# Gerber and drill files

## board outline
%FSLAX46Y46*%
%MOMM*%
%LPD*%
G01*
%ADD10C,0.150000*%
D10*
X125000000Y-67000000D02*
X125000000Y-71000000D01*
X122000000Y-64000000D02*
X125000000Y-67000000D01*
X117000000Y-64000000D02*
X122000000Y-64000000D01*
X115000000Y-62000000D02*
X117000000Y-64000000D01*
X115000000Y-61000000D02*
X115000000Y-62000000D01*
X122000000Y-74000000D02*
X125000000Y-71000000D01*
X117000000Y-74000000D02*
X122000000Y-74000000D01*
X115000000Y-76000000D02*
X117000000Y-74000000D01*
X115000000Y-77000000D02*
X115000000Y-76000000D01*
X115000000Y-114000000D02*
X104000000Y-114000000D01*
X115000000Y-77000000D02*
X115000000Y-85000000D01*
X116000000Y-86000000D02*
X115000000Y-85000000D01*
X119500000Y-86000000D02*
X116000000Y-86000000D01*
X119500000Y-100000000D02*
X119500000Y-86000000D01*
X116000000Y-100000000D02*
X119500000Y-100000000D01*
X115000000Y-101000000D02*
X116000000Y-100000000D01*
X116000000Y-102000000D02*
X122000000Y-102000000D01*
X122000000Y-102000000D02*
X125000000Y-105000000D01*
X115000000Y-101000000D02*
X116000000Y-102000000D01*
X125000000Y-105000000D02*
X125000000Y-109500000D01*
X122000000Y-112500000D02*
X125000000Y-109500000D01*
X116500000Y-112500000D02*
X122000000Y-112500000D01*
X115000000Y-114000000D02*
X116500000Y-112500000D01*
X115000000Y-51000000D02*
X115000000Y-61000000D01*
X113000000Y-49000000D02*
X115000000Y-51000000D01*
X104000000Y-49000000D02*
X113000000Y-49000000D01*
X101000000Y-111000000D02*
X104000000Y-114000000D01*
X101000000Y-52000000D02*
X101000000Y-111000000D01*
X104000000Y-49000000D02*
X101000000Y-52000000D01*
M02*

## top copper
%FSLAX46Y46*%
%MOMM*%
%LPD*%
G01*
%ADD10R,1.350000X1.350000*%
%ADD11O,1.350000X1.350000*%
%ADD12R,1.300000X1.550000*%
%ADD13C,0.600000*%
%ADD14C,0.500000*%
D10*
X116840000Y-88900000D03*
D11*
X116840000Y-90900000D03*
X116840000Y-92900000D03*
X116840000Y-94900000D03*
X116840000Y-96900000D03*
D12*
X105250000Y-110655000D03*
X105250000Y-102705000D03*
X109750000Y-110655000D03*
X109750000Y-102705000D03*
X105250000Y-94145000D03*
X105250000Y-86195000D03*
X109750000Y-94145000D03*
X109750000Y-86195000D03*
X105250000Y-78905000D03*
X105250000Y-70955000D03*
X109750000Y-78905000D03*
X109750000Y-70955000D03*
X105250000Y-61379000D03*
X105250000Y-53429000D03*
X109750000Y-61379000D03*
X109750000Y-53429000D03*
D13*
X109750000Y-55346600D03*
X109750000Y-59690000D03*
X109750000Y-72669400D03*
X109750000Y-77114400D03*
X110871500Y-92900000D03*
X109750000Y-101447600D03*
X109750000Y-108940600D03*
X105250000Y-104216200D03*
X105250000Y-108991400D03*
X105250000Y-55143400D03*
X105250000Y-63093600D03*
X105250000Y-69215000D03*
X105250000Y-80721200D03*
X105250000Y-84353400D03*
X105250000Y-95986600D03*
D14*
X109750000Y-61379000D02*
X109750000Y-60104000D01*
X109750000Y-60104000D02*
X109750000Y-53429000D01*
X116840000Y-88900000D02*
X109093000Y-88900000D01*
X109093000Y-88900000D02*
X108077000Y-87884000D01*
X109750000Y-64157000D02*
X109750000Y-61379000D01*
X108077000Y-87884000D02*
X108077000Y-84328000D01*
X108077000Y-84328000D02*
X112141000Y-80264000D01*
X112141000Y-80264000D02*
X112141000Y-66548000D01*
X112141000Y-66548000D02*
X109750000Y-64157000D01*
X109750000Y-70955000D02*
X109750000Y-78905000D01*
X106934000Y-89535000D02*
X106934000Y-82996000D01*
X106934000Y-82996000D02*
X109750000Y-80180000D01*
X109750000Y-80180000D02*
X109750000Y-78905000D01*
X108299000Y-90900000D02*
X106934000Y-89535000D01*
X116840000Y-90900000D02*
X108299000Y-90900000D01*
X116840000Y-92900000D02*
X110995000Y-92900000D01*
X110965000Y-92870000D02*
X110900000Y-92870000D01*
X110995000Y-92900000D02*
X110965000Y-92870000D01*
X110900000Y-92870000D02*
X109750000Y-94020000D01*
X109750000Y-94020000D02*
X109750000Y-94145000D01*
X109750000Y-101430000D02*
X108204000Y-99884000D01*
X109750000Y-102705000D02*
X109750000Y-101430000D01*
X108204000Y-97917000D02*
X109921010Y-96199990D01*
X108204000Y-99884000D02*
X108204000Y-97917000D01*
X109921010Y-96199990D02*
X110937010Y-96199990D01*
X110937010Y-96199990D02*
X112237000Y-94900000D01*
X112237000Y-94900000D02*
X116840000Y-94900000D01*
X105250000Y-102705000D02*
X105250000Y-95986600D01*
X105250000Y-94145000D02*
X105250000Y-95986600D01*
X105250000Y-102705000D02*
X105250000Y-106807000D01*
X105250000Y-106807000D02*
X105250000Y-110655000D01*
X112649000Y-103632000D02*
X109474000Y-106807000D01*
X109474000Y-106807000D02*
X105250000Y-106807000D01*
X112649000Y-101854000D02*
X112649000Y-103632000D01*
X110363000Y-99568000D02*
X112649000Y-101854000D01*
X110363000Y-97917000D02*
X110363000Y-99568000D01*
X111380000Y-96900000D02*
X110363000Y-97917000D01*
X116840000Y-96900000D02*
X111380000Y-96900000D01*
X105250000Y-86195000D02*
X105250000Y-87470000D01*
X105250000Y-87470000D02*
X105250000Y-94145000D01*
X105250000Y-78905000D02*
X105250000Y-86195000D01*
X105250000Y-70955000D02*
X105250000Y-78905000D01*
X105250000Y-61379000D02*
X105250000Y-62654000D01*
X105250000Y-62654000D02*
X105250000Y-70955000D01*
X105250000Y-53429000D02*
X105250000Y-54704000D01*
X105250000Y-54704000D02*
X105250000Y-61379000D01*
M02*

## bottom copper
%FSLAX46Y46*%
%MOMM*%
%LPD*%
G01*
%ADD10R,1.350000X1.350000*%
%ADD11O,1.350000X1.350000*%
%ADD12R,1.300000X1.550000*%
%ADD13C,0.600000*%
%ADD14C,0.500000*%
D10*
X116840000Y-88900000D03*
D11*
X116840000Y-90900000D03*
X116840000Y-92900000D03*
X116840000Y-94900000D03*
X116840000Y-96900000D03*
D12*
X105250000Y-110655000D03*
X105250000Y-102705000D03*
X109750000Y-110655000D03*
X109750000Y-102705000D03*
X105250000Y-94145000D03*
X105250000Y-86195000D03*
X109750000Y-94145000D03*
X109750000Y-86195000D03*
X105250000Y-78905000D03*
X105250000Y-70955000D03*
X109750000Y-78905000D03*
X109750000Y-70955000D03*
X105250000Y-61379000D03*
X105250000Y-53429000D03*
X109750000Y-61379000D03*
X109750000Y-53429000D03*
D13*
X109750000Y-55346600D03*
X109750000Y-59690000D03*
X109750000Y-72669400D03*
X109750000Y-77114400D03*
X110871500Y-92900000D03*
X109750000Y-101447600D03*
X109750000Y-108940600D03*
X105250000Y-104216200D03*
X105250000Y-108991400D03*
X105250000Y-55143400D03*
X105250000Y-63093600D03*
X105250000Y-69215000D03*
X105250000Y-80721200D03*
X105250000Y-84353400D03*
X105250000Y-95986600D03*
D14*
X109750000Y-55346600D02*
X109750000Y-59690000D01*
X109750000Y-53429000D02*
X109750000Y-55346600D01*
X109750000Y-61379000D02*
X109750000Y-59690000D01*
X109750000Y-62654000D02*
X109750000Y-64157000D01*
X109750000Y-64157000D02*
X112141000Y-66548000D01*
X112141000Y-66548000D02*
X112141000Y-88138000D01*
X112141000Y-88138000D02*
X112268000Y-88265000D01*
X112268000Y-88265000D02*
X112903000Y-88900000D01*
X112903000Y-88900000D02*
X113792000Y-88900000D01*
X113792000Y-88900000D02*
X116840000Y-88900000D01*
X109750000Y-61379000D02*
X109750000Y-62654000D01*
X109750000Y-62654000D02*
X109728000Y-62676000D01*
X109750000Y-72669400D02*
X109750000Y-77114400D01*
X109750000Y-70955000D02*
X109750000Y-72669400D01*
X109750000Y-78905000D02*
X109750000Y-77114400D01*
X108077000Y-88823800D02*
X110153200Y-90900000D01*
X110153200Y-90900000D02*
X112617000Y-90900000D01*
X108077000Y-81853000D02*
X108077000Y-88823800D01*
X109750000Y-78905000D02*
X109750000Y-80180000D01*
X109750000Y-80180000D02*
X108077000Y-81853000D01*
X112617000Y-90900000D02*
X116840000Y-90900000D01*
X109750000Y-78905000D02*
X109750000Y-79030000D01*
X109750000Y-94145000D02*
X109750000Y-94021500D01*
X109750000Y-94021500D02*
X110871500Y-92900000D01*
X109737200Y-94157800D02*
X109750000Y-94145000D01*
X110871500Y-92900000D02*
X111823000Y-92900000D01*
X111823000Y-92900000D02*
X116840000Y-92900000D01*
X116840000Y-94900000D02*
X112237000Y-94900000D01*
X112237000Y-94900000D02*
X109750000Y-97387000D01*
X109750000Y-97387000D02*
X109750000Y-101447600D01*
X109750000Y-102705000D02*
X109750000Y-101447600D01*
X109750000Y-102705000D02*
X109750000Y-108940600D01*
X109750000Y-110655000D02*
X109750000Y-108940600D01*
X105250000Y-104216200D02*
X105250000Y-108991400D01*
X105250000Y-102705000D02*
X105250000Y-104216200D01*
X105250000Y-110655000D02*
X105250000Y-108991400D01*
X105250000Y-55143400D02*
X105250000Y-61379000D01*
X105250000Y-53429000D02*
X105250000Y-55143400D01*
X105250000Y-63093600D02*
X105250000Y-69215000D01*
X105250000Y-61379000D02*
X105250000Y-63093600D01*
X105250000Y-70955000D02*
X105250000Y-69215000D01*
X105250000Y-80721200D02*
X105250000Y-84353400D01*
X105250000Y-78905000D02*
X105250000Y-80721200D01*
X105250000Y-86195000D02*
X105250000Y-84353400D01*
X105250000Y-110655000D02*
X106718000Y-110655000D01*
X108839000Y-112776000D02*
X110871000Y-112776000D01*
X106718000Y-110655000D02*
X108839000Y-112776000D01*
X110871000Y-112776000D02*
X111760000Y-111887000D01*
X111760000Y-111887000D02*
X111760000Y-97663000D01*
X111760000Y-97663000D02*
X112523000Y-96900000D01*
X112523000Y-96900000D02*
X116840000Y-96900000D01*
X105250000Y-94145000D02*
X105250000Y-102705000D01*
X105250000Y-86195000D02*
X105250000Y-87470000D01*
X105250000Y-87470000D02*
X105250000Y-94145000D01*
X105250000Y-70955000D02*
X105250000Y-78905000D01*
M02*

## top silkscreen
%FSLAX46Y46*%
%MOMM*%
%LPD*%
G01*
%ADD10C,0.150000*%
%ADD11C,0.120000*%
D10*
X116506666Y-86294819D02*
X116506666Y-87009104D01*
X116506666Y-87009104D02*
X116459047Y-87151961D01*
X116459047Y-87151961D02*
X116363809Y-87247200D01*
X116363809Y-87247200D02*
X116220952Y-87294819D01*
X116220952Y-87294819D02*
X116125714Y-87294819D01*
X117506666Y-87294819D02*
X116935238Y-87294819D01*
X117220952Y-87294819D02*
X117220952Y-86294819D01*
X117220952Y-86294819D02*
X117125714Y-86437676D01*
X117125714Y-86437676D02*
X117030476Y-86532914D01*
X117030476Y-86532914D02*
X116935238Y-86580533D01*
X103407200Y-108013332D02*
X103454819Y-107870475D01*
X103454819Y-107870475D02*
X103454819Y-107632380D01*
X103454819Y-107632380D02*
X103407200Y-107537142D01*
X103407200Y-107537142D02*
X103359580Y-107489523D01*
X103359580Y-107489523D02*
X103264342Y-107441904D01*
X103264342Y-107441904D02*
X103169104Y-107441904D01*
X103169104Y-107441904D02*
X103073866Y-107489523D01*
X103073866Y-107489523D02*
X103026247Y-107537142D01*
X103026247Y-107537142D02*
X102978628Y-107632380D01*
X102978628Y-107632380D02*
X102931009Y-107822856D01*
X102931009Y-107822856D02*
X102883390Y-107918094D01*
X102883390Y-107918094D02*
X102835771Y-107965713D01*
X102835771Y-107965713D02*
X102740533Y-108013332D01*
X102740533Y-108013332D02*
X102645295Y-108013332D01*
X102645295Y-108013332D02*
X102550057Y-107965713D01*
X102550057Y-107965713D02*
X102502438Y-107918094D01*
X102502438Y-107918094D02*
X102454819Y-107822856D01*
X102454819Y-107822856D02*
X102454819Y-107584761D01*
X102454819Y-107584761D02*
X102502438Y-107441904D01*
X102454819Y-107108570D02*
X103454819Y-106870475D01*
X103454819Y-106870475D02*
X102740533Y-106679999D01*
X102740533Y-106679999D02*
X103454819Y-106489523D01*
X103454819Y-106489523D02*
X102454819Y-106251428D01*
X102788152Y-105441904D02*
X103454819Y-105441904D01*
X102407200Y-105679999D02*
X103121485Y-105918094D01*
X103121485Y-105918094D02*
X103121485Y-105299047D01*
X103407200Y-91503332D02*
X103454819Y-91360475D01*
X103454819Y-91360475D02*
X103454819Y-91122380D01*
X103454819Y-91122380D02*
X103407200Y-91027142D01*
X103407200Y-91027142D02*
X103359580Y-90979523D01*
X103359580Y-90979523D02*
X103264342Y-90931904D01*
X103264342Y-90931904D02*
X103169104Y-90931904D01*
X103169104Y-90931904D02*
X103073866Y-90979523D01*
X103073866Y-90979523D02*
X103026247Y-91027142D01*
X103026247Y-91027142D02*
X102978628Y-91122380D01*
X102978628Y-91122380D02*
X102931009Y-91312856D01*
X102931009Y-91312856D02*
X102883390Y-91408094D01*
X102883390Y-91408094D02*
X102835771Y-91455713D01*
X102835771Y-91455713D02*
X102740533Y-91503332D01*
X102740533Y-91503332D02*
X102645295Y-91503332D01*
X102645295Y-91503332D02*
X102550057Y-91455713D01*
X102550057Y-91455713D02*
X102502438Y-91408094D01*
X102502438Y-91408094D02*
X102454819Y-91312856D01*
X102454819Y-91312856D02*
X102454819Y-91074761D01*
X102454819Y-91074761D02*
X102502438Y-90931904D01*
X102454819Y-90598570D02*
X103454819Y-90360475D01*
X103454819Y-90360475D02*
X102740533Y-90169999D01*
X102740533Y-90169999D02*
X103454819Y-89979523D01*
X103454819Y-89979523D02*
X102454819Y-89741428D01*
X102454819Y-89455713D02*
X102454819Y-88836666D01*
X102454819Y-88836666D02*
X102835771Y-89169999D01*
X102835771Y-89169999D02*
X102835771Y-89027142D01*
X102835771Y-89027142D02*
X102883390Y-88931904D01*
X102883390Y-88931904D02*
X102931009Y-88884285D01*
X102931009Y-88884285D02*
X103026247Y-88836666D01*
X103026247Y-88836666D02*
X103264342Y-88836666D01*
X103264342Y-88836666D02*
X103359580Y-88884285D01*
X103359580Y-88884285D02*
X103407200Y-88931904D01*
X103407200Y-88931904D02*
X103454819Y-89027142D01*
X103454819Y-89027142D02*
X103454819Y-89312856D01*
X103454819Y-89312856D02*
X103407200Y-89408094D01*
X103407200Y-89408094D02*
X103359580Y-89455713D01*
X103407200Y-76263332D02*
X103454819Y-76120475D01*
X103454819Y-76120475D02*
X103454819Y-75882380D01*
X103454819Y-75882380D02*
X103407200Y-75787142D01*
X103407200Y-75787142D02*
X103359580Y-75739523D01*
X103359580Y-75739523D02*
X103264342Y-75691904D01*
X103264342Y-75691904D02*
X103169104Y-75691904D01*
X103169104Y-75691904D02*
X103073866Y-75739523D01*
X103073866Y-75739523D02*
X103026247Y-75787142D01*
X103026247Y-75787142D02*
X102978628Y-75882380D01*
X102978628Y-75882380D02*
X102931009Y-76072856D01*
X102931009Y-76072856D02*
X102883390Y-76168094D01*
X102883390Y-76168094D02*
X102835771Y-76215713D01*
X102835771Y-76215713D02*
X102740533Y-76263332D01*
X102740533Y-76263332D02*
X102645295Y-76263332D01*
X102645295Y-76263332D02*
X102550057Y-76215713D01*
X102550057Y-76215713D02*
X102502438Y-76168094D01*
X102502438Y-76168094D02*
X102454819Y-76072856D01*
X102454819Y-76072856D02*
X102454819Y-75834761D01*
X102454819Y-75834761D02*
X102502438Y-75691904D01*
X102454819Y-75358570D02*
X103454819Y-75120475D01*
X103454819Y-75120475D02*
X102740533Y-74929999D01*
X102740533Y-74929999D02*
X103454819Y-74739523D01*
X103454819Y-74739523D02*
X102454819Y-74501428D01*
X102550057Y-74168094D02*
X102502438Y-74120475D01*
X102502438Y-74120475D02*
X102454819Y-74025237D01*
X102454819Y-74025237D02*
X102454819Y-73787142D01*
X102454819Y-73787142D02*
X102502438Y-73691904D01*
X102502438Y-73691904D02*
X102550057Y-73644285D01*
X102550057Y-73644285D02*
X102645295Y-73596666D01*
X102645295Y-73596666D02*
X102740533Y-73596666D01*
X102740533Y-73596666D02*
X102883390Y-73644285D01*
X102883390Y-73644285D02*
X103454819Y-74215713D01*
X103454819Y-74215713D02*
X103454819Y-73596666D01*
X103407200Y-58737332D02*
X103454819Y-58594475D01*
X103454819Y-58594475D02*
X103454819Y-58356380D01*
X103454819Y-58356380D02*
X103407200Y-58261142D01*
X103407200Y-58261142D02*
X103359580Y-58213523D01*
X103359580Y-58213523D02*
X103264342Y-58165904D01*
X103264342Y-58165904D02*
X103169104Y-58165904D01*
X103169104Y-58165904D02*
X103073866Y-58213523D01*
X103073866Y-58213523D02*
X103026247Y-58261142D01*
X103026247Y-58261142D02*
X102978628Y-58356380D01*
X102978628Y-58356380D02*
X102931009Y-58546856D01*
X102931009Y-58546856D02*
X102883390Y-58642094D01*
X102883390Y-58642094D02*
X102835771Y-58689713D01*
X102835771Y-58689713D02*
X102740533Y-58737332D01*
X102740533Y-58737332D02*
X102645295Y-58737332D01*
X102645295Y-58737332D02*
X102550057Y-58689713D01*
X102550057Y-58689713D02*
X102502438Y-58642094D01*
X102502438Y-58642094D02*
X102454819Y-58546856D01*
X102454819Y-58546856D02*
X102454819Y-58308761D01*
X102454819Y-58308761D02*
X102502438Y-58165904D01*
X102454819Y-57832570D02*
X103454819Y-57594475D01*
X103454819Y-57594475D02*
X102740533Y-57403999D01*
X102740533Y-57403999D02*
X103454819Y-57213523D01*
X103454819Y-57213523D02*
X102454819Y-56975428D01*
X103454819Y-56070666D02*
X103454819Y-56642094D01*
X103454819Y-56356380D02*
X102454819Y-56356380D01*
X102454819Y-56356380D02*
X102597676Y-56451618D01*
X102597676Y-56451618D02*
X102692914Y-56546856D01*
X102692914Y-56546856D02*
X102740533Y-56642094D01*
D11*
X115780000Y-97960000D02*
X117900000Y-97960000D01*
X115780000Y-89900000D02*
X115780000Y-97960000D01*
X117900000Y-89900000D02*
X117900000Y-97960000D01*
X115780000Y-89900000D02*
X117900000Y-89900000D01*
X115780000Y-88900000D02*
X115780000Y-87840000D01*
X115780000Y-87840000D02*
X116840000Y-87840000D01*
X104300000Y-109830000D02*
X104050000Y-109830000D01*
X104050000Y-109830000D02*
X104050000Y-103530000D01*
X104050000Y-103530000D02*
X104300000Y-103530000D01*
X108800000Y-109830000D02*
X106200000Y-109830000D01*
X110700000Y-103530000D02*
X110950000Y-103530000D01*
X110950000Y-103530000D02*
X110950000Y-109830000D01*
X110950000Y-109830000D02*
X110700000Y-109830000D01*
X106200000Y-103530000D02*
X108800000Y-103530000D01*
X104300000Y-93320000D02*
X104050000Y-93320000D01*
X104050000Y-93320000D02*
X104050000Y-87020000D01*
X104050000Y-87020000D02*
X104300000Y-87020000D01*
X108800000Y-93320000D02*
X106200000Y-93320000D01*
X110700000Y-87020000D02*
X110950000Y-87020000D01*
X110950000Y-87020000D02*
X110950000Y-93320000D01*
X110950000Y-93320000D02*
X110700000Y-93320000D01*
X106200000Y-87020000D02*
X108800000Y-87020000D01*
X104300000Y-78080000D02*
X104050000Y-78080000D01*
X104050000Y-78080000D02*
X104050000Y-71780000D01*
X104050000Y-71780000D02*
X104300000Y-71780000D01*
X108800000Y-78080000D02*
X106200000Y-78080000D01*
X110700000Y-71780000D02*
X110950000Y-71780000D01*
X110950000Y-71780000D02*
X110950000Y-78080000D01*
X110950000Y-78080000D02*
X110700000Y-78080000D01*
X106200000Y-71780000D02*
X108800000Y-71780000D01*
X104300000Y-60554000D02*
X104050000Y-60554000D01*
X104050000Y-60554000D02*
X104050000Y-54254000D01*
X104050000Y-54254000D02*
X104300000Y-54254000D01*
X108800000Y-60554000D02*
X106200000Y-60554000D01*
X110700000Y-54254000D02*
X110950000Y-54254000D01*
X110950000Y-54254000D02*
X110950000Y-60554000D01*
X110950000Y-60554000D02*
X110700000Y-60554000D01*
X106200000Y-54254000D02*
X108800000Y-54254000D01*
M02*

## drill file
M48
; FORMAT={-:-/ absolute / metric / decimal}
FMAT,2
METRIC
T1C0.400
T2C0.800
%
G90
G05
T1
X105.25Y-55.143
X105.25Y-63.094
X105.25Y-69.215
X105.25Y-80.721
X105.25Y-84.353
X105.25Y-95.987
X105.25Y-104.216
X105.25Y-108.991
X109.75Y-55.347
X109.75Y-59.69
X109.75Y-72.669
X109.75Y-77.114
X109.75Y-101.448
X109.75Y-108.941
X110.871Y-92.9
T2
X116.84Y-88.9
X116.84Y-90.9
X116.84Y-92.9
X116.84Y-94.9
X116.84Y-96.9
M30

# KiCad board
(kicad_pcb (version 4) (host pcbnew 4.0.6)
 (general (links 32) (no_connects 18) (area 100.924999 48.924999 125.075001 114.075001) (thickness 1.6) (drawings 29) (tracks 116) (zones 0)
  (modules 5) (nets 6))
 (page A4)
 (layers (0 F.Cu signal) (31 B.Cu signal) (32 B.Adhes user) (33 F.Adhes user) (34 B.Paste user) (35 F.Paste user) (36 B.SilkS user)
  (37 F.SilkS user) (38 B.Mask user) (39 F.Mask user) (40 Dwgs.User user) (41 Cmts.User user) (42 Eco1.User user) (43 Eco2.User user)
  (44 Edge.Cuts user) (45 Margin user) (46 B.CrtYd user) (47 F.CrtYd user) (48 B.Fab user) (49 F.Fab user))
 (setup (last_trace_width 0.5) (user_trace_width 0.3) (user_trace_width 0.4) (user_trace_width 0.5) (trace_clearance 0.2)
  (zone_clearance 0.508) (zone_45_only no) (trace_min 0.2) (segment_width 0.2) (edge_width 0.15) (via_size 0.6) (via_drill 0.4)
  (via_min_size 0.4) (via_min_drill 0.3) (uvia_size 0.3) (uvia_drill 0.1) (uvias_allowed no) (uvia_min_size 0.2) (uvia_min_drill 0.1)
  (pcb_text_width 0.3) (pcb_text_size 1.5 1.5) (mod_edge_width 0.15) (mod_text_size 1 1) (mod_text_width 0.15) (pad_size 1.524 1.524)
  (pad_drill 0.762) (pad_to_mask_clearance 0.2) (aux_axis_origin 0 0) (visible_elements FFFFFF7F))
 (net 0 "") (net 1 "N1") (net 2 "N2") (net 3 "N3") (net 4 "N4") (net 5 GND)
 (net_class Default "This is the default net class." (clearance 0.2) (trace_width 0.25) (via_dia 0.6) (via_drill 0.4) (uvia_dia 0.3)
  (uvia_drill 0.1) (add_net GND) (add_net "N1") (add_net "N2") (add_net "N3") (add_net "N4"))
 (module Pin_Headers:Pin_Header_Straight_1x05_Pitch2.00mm (layer F.Cu) (at 116.84 88.9)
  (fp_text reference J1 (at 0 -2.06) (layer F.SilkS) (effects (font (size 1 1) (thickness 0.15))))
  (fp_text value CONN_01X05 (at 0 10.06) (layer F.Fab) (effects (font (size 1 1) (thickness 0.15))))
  (fp_line (start -1.06 9.06) (end 1.06 9.06) (layer F.SilkS) (width 0.12))
  (fp_line (start -1.06 1) (end -1.06 9.06) (layer F.SilkS) (width 0.12))
  (fp_line (start 1.06 1) (end 1.06 9.06) (layer F.SilkS) (width 0.12))
  (fp_line (start -1.06 1) (end 1.06 1) (layer F.SilkS) (width 0.12))
  (fp_line (start -1.06 0) (end -1.06 -1.06) (layer F.SilkS) (width 0.12))
  (fp_line (start -1.06 -1.06) (end 0 -1.06) (layer F.SilkS) (width 0.12))
  (pad 1 thru_hole rect (at 0 0) (size 1.35 1.35) (drill 0.8) (layers *.Cu *.Mask) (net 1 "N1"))
  (pad 2 thru_hole oval (at 0 2) (size 1.35 1.35) (drill 0.8) (layers *.Cu *.Mask) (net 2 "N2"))
  (pad 3 thru_hole oval (at 0 4) (size 1.35 1.35) (drill 0.8) (layers *.Cu *.Mask) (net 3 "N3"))
  (pad 4 thru_hole oval (at 0 6) (size 1.35 1.35) (drill 0.8) (layers *.Cu *.Mask) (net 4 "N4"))
  (pad 5 thru_hole oval (at 0 8) (size 1.35 1.35) (drill 0.8) (layers *.Cu *.Mask) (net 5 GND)))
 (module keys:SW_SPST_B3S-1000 (layer F.Cu) (at 107.5 106.68 90)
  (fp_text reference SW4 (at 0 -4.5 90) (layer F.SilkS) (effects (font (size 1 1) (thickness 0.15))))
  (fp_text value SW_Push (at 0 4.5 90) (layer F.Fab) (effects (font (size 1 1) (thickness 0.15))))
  (fp_line (start -3.15 -3.2) (end -3.15 -3.45) (layer F.SilkS) (width 0.12))
  (fp_line (start -3.15 -3.45) (end 3.15 -3.45) (layer F.SilkS) (width 0.12))
  (fp_line (start 3.15 -3.45) (end 3.15 -3.2) (layer F.SilkS) (width 0.12))
  (fp_line (start -3.15 1.3) (end -3.15 -1.3) (layer F.SilkS) (width 0.12))
  (fp_line (start 3.15 3.2) (end 3.15 3.45) (layer F.SilkS) (width 0.12))
  (fp_line (start 3.15 3.45) (end -3.15 3.45) (layer F.SilkS) (width 0.12))
  (fp_line (start -3.15 3.45) (end -3.15 3.2) (layer F.SilkS) (width 0.12))
  (fp_line (start 3.15 -1.3) (end 3.15 1.3) (layer F.SilkS) (width 0.12))
  (pad 1 smd rect (at -3.975 -2.25 90) (size 1.55 1.3) (layers F.Cu F.Paste F.Mask) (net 5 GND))
  (pad 1 smd rect (at 3.975 -2.25 90) (size 1.55 1.3) (layers F.Cu F.Paste F.Mask) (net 5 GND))
  (pad 2 smd rect (at -3.975 2.25 90) (size 1.55 1.3) (layers F.Cu F.Paste F.Mask) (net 4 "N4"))
  (pad 2 smd rect (at 3.975 2.25 90) (size 1.55 1.3) (layers F.Cu F.Paste F.Mask) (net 4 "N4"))
  (pad 1 smd rect (at -3.975 -2.25 90) (size 1.55 1.3) (layers B.Cu B.Paste B.Mask) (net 5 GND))
  (pad 1 smd rect (at 3.975 -2.25 90) (size 1.55 1.3) (layers B.Cu B.Paste B.Mask) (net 5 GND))
  (pad 2 smd rect (at -3.975 2.25 90) (size 1.55 1.3) (layers B.Cu B.Paste B.Mask) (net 4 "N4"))
  (pad 2 smd rect (at 3.975 2.25 90) (size 1.55 1.3) (layers B.Cu B.Paste B.Mask) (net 4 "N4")))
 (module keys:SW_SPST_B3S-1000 (layer F.Cu) (at 107.5 90.17 90)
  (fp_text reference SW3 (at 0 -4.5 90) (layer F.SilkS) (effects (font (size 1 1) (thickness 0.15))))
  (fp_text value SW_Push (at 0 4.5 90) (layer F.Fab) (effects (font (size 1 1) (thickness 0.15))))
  (fp_line (start -3.15 -3.2) (end -3.15 -3.45) (layer F.SilkS) (width 0.12))
  (fp_line (start -3.15 -3.45) (end 3.15 -3.45) (layer F.SilkS) (width 0.12))
  (fp_line (start 3.15 -3.45) (end 3.15 -3.2) (layer F.SilkS) (width 0.12))
  (fp_line (start -3.15 1.3) (end -3.15 -1.3) (layer F.SilkS) (width 0.12))
  (fp_line (start 3.15 3.2) (end 3.15 3.45) (layer F.SilkS) (width 0.12))
  (fp_line (start 3.15 3.45) (end -3.15 3.45) (layer F.SilkS) (width 0.12))
  (fp_line (start -3.15 3.45) (end -3.15 3.2) (layer F.SilkS) (width 0.12))
  (fp_line (start 3.15 -1.3) (end 3.15 1.3) (layer F.SilkS) (width 0.12))
  (pad 1 smd rect (at -3.975 -2.25 90) (size 1.55 1.3) (layers F.Cu F.Paste F.Mask) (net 5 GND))
  (pad 1 smd rect (at 3.975 -2.25 90) (size 1.55 1.3) (layers F.Cu F.Paste F.Mask) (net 5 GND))
  (pad 2 smd rect (at -3.975 2.25 90) (size 1.55 1.3) (layers F.Cu F.Paste F.Mask) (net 3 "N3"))
  (pad 2 smd rect (at 3.975 2.25 90) (size 1.55 1.3) (layers F.Cu F.Paste F.Mask) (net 3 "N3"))
  (pad 1 smd rect (at -3.975 -2.25 90) (size 1.55 1.3) (layers B.Cu B.Paste B.Mask) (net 5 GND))
  (pad 1 smd rect (at 3.975 -2.25 90) (size 1.55 1.3) (layers B.Cu B.Paste B.Mask) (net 5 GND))
  (pad 2 smd rect (at -3.975 2.25 90) (size 1.55 1.3) (layers B.Cu B.Paste B.Mask) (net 3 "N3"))
  (pad 2 smd rect (at 3.975 2.25 90) (size 1.55 1.3) (layers B.Cu B.Paste B.Mask) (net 3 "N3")))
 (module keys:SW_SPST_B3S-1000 (layer F.Cu) (at 107.5 74.93 90)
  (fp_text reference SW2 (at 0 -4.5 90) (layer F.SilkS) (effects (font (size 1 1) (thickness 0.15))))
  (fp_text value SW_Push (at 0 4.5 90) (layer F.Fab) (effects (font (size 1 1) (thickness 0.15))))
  (fp_line (start -3.15 -3.2) (end -3.15 -3.45) (layer F.SilkS) (width 0.12))
  (fp_line (start -3.15 -3.45) (end 3.15 -3.45) (layer F.SilkS) (width 0.12))
  (fp_line (start 3.15 -3.45) (end 3.15 -3.2) (layer F.SilkS) (width 0.12))
  (fp_line (start -3.15 1.3) (end -3.15 -1.3) (layer F.SilkS) (width 0.12))
  (fp_line (start 3.15 3.2) (end 3.15 3.45) (layer F.SilkS) (width 0.12))
  (fp_line (start 3.15 3.45) (end -3.15 3.45) (layer F.SilkS) (width 0.12))
  (fp_line (start -3.15 3.45) (end -3.15 3.2) (layer F.SilkS) (width 0.12))
  (fp_line (start 3.15 -1.3) (end 3.15 1.3) (layer F.SilkS) (width 0.12))
  (pad 1 smd rect (at -3.975 -2.25 90) (size 1.55 1.3) (layers F.Cu F.Paste F.Mask) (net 5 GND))
  (pad 1 smd rect (at 3.975 -2.25 90) (size 1.55 1.3) (layers F.Cu F.Paste F.Mask) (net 5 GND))
  (pad 2 smd rect (at -3.975 2.25 90) (size 1.55 1.3) (layers F.Cu F.Paste F.Mask) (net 2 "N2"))
  (pad 2 smd rect (at 3.975 2.25 90) (size 1.55 1.3) (layers F.Cu F.Paste F.Mask) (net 2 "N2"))
  (pad 1 smd rect (at -3.975 -2.25 90) (size 1.55 1.3) (layers B.Cu B.Paste B.Mask) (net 5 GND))
  (pad 1 smd rect (at 3.975 -2.25 90) (size 1.55 1.3) (layers B.Cu B.Paste B.Mask) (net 5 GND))
  (pad 2 smd rect (at -3.975 2.25 90) (size 1.55 1.3) (layers B.Cu B.Paste B.Mask) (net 2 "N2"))
  (pad 2 smd rect (at 3.975 2.25 90) (size 1.55 1.3) (layers B.Cu B.Paste B.Mask) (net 2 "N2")))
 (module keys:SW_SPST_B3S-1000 (layer F.Cu) (at 107.5 57.404 90)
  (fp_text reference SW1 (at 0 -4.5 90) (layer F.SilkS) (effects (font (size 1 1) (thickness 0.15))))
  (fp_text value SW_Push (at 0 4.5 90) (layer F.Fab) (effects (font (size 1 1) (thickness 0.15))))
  (fp_line (start -3.15 -3.2) (end -3.15 -3.45) (layer F.SilkS) (width 0.12))
  (fp_line (start -3.15 -3.45) (end 3.15 -3.45) (layer F.SilkS) (width 0.12))
  (fp_line (start 3.15 -3.45) (end 3.15 -3.2) (layer F.SilkS) (width 0.12))
  (fp_line (start -3.15 1.3) (end -3.15 -1.3) (layer F.SilkS) (width 0.12))
  (fp_line (start 3.15 3.2) (end 3.15 3.45) (layer F.SilkS) (width 0.12))
  (fp_line (start 3.15 3.45) (end -3.15 3.45) (layer F.SilkS) (width 0.12))
  (fp_line (start -3.15 3.45) (end -3.15 3.2) (layer F.SilkS) (width 0.12))
  (fp_line (start 3.15 -1.3) (end 3.15 1.3) (layer F.SilkS) (width 0.12))
  (pad 1 smd rect (at -3.975 -2.25 90) (size 1.55 1.3) (layers F.Cu F.Paste F.Mask) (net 5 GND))
  (pad 1 smd rect (at 3.975 -2.25 90) (size 1.55 1.3) (layers F.Cu F.Paste F.Mask) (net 5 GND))
  (pad 2 smd rect (at -3.975 2.25 90) (size 1.55 1.3) (layers F.Cu F.Paste F.Mask) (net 1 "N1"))
  (pad 2 smd rect (at 3.975 2.25 90) (size 1.55 1.3) (layers F.Cu F.Paste F.Mask) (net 1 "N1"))
  (pad 1 smd rect (at -3.975 -2.25 90) (size 1.55 1.3) (layers B.Cu B.Paste B.Mask) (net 5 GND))
  (pad 1 smd rect (at 3.975 -2.25 90) (size 1.55 1.3) (layers B.Cu B.Paste B.Mask) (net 5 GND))
  (pad 2 smd rect (at -3.975 2.25 90) (size 1.55 1.3) (layers B.Cu B.Paste B.Mask) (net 1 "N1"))
  (pad 2 smd rect (at 3.975 2.25 90) (size 1.55 1.3) (layers B.Cu B.Paste B.Mask) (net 1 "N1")))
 (gr_line (start 125 67) (end 125 71) (layer Edge.Cuts) (width 0.15))
 (gr_line (start 122 64) (end 125 67) (layer Edge.Cuts) (width 0.15))
 (gr_line (start 117 64) (end 122 64) (layer Edge.Cuts) (width 0.15))
 (gr_line (start 115 62) (end 117 64) (layer Edge.Cuts) (width 0.15))
 (gr_line (start 115 61) (end 115 62) (layer Edge.Cuts) (width 0.15))
 (gr_line (start 122 74) (end 125 71) (layer Edge.Cuts) (width 0.15))
 (gr_line (start 117 74) (end 122 74) (layer Edge.Cuts) (width 0.15))
 (gr_line (start 115 76) (end 117 74) (layer Edge.Cuts) (width 0.15))
 (gr_line (start 115 77) (end 115 76) (layer Edge.Cuts) (width 0.15))
 (gr_line (start 115 114) (end 104 114) (layer Edge.Cuts) (width 0.15))
 (gr_line (start 115 77) (end 115 85) (layer Edge.Cuts) (width 0.15))
 (gr_line (start 116 86) (end 115 85) (layer Edge.Cuts) (width 0.15))
 (gr_line (start 119.5 86) (end 116 86) (layer Edge.Cuts) (width 0.15))
 (gr_line (start 119.5 100) (end 119.5 86) (layer Edge.Cuts) (width 0.15))
 (gr_line (start 116 100) (end 119.5 100) (layer Edge.Cuts) (width 0.15))
 (gr_line (start 115 101) (end 116 100) (layer Edge.Cuts) (width 0.15))
 (gr_line (start 116 102) (end 122 102) (layer Edge.Cuts) (width 0.15))
 (gr_line (start 122 102) (end 125 105) (layer Edge.Cuts) (width 0.15))
 (gr_line (start 115 101) (end 116 102) (layer Edge.Cuts) (width 0.15))
 (gr_line (start 125 105) (end 125 109.5) (layer Edge.Cuts) (width 0.15))
 (gr_line (start 122 112.5) (end 125 109.5) (layer Edge.Cuts) (width 0.15))
 (gr_line (start 116.5 112.5) (end 122 112.5) (layer Edge.Cuts) (width 0.15))
 (gr_line (start 115 114) (end 116.5 112.5) (layer Edge.Cuts) (width 0.15))
 (gr_line (start 115 51) (end 115 61) (layer Edge.Cuts) (width 0.15))
 (gr_line (start 113 49) (end 115 51) (layer Edge.Cuts) (width 0.15))
 (gr_line (start 104 49) (end 113 49) (layer Edge.Cuts) (width 0.15))
 (gr_line (start 101 111) (end 104 114) (layer Edge.Cuts) (width 0.15))
 (gr_line (start 101 52) (end 101 111) (layer Edge.Cuts) (width 0.15))
 (gr_line (start 104 49) (end 101 52) (layer Edge.Cuts) (width 0.15))
 (segment (start 109.75 55.3466) (end 109.75 59.69) (width 0.5) (layer B.Cu) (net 1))
 (segment (start 109.75 53.429) (end 109.75 55.3466) (width 0.5) (layer B.Cu) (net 1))
 (via (at 109.75 55.3466) (size 0.6) (drill 0.4) (layers F.Cu B.Cu) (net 1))
 (segment (start 109.75 61.379) (end 109.75 59.69) (width 0.5) (layer B.Cu) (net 1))
 (via (at 109.75 59.69) (size 0.6) (drill 0.4) (layers F.Cu B.Cu) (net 1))
 (segment (start 109.75 62.654) (end 109.75 64.157) (width 0.5) (layer B.Cu) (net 1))
 (segment (start 109.75 64.157) (end 112.141 66.548) (width 0.5) (layer B.Cu) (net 1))
 (segment (start 112.141 66.548) (end 112.141 88.138) (width 0.5) (layer B.Cu) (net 1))
 (segment (start 112.141 88.138) (end 112.268 88.265) (width 0.5) (layer B.Cu) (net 1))
 (segment (start 112.268 88.265) (end 112.903 88.9) (width 0.5) (layer B.Cu) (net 1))
 (segment (start 112.903 88.9) (end 113.792 88.9) (width 0.5) (layer B.Cu) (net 1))
 (segment (start 113.792 88.9) (end 116.84 88.9) (width 0.5) (layer B.Cu) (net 1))
 (segment (start 109.75 61.379) (end 109.75 62.654) (width 0.5) (layer B.Cu) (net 1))
 (segment (start 109.75 62.654) (end 109.728 62.676) (width 0.5) (layer B.Cu) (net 1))
 (segment (start 109.75 61.379) (end 109.75 60.104) (width 0.5) (layer F.Cu) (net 1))
 (segment (start 109.75 60.104) (end 109.75 53.429) (width 0.5) (layer F.Cu) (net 1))
 (segment (start 116.84 88.9) (end 109.093 88.9) (width 0.5) (layer F.Cu) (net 1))
 (segment (start 109.093 88.9) (end 108.077 87.884) (width 0.5) (layer F.Cu) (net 1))
 (segment (start 109.75 64.157) (end 109.75 61.379) (width 0.5) (layer F.Cu) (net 1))
 (segment (start 108.077 87.884) (end 108.077 84.328) (width 0.5) (layer F.Cu) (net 1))
 (segment (start 108.077 84.328) (end 112.141 80.264) (width 0.5) (layer F.Cu) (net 1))
 (segment (start 112.141 80.264) (end 112.141 66.548) (width 0.5) (layer F.Cu) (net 1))
 (segment (start 112.141 66.548) (end 109.75 64.157) (width 0.5) (layer F.Cu) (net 1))
 (segment (start 109.75 72.6694) (end 109.75 77.1144) (width 0.5) (layer B.Cu) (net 2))
 (segment (start 109.75 70.955) (end 109.75 72.6694) (width 0.5) (layer B.Cu) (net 2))
 (via (at 109.75 72.6694) (size 0.6) (drill 0.4) (layers F.Cu B.Cu) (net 2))
 (segment (start 109.75 78.905) (end 109.75 77.1144) (width 0.5) (layer B.Cu) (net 2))
 (via (at 109.75 77.1144) (size 0.6) (drill 0.4) (layers F.Cu B.Cu) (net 2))
 (segment (start 108.077 88.8238) (end 110.1532 90.9) (width 0.5) (layer B.Cu) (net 2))
 (segment (start 110.1532 90.9) (end 112.617 90.9) (width 0.5) (layer B.Cu) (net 2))
 (segment (start 108.077 81.853) (end 108.077 88.8238) (width 0.5) (layer B.Cu) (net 2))
 (segment (start 109.75 78.905) (end 109.75 80.18) (width 0.5) (layer B.Cu) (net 2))
 (segment (start 109.75 80.18) (end 108.077 81.853) (width 0.5) (layer B.Cu) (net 2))
 (segment (start 112.617 90.9) (end 116.84 90.9) (width 0.5) (layer B.Cu) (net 2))
 (segment (start 109.75 78.905) (end 109.75 79.03) (width 0.5) (layer B.Cu) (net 2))
 (segment (start 109.75 70.955) (end 109.75 78.905) (width 0.5) (layer F.Cu) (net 2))
 (segment (start 106.934 89.535) (end 106.934 82.996) (width 0.5) (layer F.Cu) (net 2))
 (segment (start 106.934 82.996) (end 109.75 80.18) (width 0.5) (layer F.Cu) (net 2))
 (segment (start 109.75 80.18) (end 109.75 78.905) (width 0.5) (layer F.Cu) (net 2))
 (segment (start 108.299 90.9) (end 106.934 89.535) (width 0.5) (layer F.Cu) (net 2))
 (segment (start 116.84 90.9) (end 108.299 90.9) (width 0.5) (layer F.Cu) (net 2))
 (segment (start 109.75 94.145) (end 109.75 94.0215) (width 0.5) (layer B.Cu) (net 3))
 (segment (start 109.75 94.0215) (end 110.8715 92.9) (width 0.5) (layer B.Cu) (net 3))
 (via (at 110.8715 92.9) (size 0.6) (drill 0.4) (layers F.Cu B.Cu) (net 3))
 (segment (start 109.7372 94.1578) (end 109.75 94.145) (width 0.5) (layer B.Cu) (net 3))
 (segment (start 110.8715 92.9) (end 111.823 92.9) (width 0.5) (layer B.Cu) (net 3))
 (segment (start 111.823 92.9) (end 116.84 92.9) (width 0.5) (layer B.Cu) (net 3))
 (segment (start 116.84 92.9) (end 110.995 92.9) (width 0.5) (layer F.Cu) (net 3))
 (segment (start 110.965 92.87) (end 110.9 92.87) (width 0.5) (layer F.Cu) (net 3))
 (segment (start 110.995 92.9) (end 110.965 92.87) (width 0.5) (layer F.Cu) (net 3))
 (segment (start 110.9 92.87) (end 109.75 94.02) (width 0.5) (layer F.Cu) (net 3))
 (segment (start 109.75 94.02) (end 109.75 94.145) (width 0.5) (layer F.Cu) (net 3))
 (segment (start 116.84 94.9) (end 112.237 94.9) (width 0.5) (layer B.Cu) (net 4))
 (segment (start 112.237 94.9) (end 109.75 97.387) (width 0.5) (layer B.Cu) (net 4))
 (segment (start 109.75 97.387) (end 109.75 101.4476) (width 0.5) (layer B.Cu) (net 4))
 (segment (start 109.75 102.705) (end 109.75 101.4476) (width 0.5) (layer B.Cu) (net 4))
 (via (at 109.75 101.4476) (size 0.6) (drill 0.4) (layers F.Cu B.Cu) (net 4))
 (segment (start 109.75 102.705) (end 109.75 108.9406) (width 0.5) (layer B.Cu) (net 4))
 (segment (start 109.75 110.655) (end 109.75 108.9406) (width 0.5) (layer B.Cu) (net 4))
 (via (at 109.75 108.9406) (size 0.6) (drill 0.4) (layers F.Cu B.Cu) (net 4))
 (segment (start 109.75 101.43) (end 108.204 99.884) (width 0.5) (layer F.Cu) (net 4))
 (segment (start 109.75 102.705) (end 109.75 101.43) (width 0.5) (layer F.Cu) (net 4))
 (segment (start 108.204 97.917) (end 109.92101 96.19999) (width 0.5) (layer F.Cu) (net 4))
 (segment (start 108.204 99.884) (end 108.204 97.917) (width 0.5) (layer F.Cu) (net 4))
 (segment (start 109.92101 96.19999) (end 110.93701 96.19999) (width 0.5) (layer F.Cu) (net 4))
 (segment (start 110.93701 96.19999) (end 112.237 94.9) (width 0.5) (layer F.Cu) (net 4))
 (segment (start 112.237 94.9) (end 116.84 94.9) (width 0.5) (layer F.Cu) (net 4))
 (segment (start 105.25 104.2162) (end 105.25 108.9914) (width 0.5) (layer B.Cu) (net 5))
 (segment (start 105.25 102.705) (end 105.25 104.2162) (width 0.5) (layer B.Cu) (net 5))
 (via (at 105.25 104.2162) (size 0.6) (drill 0.4) (layers F.Cu B.Cu) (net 5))
 (segment (start 105.25 110.655) (end 105.25 108.9914) (width 0.5) (layer B.Cu) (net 5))
 (via (at 105.25 108.9914) (size 0.6) (drill 0.4) (layers F.Cu B.Cu) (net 5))
 (segment (start 105.25 55.1434) (end 105.25 61.379) (width 0.5) (layer B.Cu) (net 5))
 (via (at 105.25 55.1434) (size 0.6) (drill 0.4) (layers F.Cu B.Cu) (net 5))
 (segment (start 105.25 53.429) (end 105.25 55.1434) (width 0.5) (layer B.Cu) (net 5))
 (segment (start 105.25 63.0936) (end 105.25 69.215) (width 0.5) (layer B.Cu) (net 5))
 (segment (start 105.25 61.379) (end 105.25 63.0936) (width 0.5) (layer B.Cu) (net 5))
 (via (at 105.25 63.0936) (size 0.6) (drill 0.4) (layers F.Cu B.Cu) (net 5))
 (segment (start 105.25 70.955) (end 105.25 69.215) (width 0.5) (layer B.Cu) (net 5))
 (via (at 105.25 69.215) (size 0.6) (drill 0.4) (layers F.Cu B.Cu) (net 5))
 (segment (start 105.25 80.7212) (end 105.25 84.3534) (width 0.5) (layer B.Cu) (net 5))
 (segment (start 105.25 78.905) (end 105.25 80.7212) (width 0.5) (layer B.Cu) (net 5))
 (via (at 105.25 80.7212) (size 0.6) (drill 0.4) (layers F.Cu B.Cu) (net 5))
 (segment (start 105.25 86.195) (end 105.25 84.3534) (width 0.5) (layer B.Cu) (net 5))
 (via (at 105.25 84.3534) (size 0.6) (drill 0.4) (layers F.Cu B.Cu) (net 5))
 (segment (start 105.25 102.705) (end 105.25 95.9866) (width 0.5) (layer F.Cu) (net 5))
 (segment (start 105.25 94.145) (end 105.25 95.9866) (width 0.5) (layer F.Cu) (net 5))
 (via (at 105.25 95.9866) (size 0.6) (drill 0.4) (layers F.Cu B.Cu) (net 5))
 (segment (start 105.25 110.655) (end 106.718 110.655) (width 0.5) (layer B.Cu) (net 5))
 (segment (start 108.839 112.776) (end 110.871 112.776) (width 0.5) (layer B.Cu) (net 5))
 (segment (start 106.718 110.655) (end 108.839 112.776) (width 0.5) (layer B.Cu) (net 5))
 (segment (start 110.871 112.776) (end 111.76 111.887) (width 0.5) (layer B.Cu) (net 5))
 (segment (start 111.76 111.887) (end 111.76 97.663) (width 0.5) (layer B.Cu) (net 5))
 (segment (start 111.76 97.663) (end 112.523 96.9) (width 0.5) (layer B.Cu) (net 5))
 (segment (start 112.523 96.9) (end 116.84 96.9) (width 0.5) (layer B.Cu) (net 5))
 (segment (start 105.25 94.145) (end 105.25 102.705) (width 0.5) (layer B.Cu) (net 5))
 (segment (start 105.25 86.195) (end 105.25 87.47) (width 0.5) (layer B.Cu) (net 5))
 (segment (start 105.25 87.47) (end 105.25 94.145) (width 0.5) (layer B.Cu) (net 5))
 (segment (start 105.25 70.955) (end 105.25 78.905) (width 0.5) (layer B.Cu) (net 5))
 (segment (start 105.25 102.705) (end 105.25 106.807) (width 0.5) (layer F.Cu) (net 5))
 (segment (start 105.25 106.807) (end 105.25 110.655) (width 0.5) (layer F.Cu) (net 5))
 (segment (start 112.649 103.632) (end 109.474 106.807) (width 0.5) (layer F.Cu) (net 5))
 (segment (start 109.474 106.807) (end 105.25 106.807) (width 0.5) (layer F.Cu) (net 5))
 (segment (start 112.649 101.854) (end 112.649 103.632) (width 0.5) (layer F.Cu) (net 5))
 (segment (start 110.363 99.568) (end 112.649 101.854) (width 0.5) (layer F.Cu) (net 5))
 (segment (start 110.363 97.917) (end 110.363 99.568) (width 0.5) (layer F.Cu) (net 5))
 (segment (start 111.38 96.9) (end 110.363 97.917) (width 0.5) (layer F.Cu) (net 5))
 (segment (start 116.84 96.9) (end 111.38 96.9) (width 0.5) (layer F.Cu) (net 5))
 (segment (start 105.25 86.195) (end 105.25 87.47) (width 0.5) (layer F.Cu) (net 5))
 (segment (start 105.25 87.47) (end 105.25 94.145) (width 0.5) (layer F.Cu) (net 5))
 (segment (start 105.25 78.905) (end 105.25 86.195) (width 0.5) (layer F.Cu) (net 5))
 (segment (start 105.25 70.955) (end 105.25 78.905) (width 0.5) (layer F.Cu) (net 5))
 (segment (start 105.25 61.379) (end 105.25 62.654) (width 0.5) (layer F.Cu) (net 5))
 (segment (start 105.25 62.654) (end 105.25 70.955) (width 0.5) (layer F.Cu) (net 5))
 (segment (start 105.25 53.429) (end 105.25 54.704) (width 0.5) (layer F.Cu) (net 5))
 (segment (start 105.25 54.704) (end 105.25 61.379) (width 0.5) (layer F.Cu) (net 5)))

